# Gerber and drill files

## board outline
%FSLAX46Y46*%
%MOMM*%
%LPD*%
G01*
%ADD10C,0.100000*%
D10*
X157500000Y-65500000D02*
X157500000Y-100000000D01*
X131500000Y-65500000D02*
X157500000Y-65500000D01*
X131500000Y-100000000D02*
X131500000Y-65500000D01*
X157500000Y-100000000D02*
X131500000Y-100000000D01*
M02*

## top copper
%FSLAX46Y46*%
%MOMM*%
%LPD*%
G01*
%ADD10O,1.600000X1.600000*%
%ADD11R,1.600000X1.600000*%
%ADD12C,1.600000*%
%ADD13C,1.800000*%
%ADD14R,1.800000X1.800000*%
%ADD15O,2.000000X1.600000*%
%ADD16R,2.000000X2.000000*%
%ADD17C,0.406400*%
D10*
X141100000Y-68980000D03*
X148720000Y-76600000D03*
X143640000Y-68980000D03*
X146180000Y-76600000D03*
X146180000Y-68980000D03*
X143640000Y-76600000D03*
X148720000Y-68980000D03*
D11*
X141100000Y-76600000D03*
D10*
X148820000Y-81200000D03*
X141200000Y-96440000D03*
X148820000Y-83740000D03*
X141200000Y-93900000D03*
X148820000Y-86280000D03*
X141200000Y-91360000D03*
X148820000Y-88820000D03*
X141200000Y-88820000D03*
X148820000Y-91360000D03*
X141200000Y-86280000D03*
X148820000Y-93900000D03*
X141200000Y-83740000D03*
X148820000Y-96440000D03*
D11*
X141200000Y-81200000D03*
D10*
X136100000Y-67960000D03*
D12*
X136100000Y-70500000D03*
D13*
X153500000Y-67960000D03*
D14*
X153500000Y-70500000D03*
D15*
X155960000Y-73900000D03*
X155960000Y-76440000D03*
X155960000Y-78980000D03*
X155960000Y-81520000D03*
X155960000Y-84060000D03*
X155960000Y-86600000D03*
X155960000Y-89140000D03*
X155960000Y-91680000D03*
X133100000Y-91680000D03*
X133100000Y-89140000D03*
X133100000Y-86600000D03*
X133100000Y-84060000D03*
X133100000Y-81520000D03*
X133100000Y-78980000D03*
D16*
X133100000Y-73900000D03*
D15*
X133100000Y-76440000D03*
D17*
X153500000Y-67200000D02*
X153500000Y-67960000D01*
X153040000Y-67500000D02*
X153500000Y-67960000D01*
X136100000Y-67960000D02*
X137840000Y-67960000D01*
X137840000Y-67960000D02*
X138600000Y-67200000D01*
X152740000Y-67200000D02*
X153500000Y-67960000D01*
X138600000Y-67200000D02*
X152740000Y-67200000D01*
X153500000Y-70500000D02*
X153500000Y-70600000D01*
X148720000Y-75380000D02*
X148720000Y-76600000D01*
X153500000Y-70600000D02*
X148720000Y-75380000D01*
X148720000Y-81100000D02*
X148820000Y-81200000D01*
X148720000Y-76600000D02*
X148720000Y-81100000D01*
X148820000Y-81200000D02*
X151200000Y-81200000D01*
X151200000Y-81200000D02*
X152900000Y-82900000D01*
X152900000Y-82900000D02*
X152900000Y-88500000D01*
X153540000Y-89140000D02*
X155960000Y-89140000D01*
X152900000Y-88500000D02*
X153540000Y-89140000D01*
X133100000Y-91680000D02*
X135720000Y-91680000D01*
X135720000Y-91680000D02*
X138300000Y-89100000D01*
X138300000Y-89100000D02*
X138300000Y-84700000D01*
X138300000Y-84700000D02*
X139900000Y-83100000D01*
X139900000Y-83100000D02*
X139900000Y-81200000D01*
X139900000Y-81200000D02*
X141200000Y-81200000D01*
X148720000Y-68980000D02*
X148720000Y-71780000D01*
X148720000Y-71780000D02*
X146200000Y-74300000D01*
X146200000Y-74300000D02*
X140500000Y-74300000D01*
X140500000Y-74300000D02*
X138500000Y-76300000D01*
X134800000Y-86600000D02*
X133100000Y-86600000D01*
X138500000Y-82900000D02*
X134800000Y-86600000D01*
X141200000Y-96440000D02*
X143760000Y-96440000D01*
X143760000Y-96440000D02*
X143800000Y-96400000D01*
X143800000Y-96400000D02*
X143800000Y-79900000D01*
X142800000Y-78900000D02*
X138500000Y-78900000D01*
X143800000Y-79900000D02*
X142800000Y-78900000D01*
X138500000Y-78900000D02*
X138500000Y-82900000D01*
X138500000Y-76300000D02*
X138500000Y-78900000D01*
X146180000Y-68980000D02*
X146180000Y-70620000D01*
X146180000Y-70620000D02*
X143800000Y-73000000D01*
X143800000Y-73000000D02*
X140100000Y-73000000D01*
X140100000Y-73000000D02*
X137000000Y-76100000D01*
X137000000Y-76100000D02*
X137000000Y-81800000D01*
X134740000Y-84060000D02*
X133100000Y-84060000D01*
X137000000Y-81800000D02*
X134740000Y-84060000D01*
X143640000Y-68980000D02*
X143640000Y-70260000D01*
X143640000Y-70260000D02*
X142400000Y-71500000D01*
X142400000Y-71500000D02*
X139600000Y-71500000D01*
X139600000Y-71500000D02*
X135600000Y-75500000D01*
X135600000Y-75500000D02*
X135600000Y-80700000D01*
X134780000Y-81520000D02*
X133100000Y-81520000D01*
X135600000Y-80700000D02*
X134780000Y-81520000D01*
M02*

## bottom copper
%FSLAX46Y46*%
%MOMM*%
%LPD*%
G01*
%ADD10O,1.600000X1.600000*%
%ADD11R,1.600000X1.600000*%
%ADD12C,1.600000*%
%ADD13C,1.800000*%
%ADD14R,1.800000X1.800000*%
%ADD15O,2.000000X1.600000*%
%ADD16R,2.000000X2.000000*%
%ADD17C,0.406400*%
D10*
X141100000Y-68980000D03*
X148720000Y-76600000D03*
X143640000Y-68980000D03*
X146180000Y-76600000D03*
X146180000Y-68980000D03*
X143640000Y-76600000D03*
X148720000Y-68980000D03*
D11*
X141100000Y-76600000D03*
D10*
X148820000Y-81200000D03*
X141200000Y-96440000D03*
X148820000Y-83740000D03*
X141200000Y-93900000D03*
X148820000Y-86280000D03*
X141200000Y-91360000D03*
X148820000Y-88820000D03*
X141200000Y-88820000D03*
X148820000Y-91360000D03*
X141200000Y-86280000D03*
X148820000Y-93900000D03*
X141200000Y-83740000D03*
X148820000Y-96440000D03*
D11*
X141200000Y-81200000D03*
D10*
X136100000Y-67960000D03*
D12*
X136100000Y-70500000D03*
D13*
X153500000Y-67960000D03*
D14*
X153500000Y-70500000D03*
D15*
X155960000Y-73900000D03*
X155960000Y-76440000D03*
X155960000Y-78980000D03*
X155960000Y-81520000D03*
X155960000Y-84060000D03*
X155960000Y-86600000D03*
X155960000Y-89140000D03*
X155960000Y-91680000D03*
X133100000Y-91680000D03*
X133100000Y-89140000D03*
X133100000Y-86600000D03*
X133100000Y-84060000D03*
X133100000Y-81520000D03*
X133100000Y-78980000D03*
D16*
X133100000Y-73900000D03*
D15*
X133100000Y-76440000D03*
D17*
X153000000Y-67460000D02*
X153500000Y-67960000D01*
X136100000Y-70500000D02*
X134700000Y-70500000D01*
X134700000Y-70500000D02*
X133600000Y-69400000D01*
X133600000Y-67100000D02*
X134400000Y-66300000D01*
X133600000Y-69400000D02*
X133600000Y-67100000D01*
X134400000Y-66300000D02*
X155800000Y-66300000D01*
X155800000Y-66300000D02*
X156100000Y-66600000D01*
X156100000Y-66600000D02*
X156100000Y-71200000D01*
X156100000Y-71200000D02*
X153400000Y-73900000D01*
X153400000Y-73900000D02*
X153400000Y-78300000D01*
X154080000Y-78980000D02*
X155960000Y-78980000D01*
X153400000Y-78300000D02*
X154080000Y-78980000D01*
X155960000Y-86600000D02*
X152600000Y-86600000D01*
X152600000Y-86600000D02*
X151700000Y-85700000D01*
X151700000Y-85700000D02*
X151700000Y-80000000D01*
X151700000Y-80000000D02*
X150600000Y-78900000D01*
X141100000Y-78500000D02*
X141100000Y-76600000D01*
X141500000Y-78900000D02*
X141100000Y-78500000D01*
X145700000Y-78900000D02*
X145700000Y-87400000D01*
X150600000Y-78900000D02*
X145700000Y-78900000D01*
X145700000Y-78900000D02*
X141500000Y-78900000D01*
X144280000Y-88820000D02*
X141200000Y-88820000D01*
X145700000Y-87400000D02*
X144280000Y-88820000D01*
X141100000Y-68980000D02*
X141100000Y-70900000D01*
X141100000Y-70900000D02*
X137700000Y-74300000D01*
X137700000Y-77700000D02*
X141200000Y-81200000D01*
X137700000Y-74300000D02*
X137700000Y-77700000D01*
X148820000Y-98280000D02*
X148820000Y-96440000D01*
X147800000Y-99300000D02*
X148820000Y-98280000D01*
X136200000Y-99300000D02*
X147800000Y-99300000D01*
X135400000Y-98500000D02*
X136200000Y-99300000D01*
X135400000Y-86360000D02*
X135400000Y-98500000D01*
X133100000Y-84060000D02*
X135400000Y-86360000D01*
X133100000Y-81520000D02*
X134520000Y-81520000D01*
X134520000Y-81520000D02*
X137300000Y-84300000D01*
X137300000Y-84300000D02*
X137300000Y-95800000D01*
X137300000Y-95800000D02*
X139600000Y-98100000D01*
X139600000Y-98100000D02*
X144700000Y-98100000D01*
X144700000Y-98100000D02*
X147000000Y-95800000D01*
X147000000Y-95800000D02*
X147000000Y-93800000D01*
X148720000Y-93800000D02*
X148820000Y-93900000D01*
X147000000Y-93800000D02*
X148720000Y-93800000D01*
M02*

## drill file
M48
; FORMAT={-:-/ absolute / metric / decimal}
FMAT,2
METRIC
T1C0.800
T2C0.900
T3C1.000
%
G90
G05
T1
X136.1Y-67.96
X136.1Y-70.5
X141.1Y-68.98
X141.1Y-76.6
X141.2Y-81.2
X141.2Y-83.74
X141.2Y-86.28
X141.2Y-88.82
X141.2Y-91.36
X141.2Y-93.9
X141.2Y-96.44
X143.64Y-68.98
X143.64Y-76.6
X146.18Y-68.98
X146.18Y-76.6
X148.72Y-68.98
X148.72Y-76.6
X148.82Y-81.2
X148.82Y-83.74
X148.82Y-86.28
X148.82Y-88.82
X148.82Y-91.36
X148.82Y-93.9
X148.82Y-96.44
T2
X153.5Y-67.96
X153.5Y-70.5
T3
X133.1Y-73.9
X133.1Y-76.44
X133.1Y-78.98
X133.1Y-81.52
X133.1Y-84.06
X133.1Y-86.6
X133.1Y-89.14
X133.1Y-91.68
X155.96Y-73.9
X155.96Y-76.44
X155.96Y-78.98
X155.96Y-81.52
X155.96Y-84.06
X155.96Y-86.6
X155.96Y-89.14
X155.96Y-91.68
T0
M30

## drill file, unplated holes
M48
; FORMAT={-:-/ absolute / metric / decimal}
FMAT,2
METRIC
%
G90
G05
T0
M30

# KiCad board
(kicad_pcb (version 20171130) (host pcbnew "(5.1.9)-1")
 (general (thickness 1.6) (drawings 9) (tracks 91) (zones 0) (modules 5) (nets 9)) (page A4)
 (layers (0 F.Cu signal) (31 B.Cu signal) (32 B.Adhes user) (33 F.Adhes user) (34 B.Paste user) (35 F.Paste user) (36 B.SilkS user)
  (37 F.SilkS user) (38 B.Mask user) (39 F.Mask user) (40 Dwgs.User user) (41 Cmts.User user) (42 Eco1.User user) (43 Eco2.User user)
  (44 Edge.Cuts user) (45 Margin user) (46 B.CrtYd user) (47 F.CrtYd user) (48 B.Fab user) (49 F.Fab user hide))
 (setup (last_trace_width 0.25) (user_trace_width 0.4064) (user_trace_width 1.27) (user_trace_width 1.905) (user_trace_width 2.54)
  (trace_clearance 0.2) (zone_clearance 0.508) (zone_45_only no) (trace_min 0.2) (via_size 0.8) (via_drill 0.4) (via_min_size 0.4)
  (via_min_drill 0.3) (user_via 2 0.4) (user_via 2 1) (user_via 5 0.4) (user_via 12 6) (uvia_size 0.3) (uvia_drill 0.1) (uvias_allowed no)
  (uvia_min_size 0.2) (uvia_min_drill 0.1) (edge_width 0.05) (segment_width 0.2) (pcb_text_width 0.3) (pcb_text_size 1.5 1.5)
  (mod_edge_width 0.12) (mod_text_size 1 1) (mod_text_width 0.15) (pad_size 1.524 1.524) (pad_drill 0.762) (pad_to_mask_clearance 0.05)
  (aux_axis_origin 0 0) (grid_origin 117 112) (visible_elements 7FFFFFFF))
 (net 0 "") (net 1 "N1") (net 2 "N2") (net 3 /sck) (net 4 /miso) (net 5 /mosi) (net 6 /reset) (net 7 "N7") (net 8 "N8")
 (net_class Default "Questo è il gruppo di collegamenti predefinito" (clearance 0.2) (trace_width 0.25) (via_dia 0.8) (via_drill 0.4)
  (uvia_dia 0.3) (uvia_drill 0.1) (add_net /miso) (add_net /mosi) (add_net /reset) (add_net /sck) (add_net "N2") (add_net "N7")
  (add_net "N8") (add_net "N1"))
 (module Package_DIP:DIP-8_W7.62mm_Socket (layer F.Cu) (at 141.1 76.6 90)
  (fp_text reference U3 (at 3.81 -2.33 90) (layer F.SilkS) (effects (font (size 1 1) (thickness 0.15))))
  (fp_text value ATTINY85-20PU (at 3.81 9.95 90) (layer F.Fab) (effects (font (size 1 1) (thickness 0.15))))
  (pad 8 thru_hole oval (at 7.62 0 90) (size 1.6 1.6) (drill 0.8) (layers *.Cu *.Mask) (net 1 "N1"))
  (pad 4 thru_hole oval (at 0 7.62 90) (size 1.6 1.6) (drill 0.8) (layers *.Cu *.Mask) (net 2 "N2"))
  (pad 7 thru_hole oval (at 7.62 2.54 90) (size 1.6 1.6) (drill 0.8) (layers *.Cu *.Mask) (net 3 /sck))
  (pad 3 thru_hole oval (at 0 5.08 90) (size 1.6 1.6) (drill 0.8) (layers *.Cu *.Mask))
  (pad 6 thru_hole oval (at 7.62 5.08 90) (size 1.6 1.6) (drill 0.8) (layers *.Cu *.Mask) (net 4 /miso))
  (pad 2 thru_hole oval (at 0 2.54 90) (size 1.6 1.6) (drill 0.8) (layers *.Cu *.Mask))
  (pad 5 thru_hole oval (at 7.62 7.62 90) (size 1.6 1.6) (drill 0.8) (layers *.Cu *.Mask) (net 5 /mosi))
  (pad 1 thru_hole rect (at 0 0 90) (size 1.6 1.6) (drill 0.8) (layers *.Cu *.Mask) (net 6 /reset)))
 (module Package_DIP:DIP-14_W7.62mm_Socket (layer F.Cu) (at 141.2 81.2)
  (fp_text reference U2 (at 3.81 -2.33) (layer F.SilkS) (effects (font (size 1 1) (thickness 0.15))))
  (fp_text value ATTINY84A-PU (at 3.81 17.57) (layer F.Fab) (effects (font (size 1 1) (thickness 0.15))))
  (pad 14 thru_hole oval (at 7.62 0) (size 1.6 1.6) (drill 0.8) (layers *.Cu *.Mask) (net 2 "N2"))
  (pad 7 thru_hole oval (at 0 15.24) (size 1.6 1.6) (drill 0.8) (layers *.Cu *.Mask) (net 5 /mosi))
  (pad 13 thru_hole oval (at 7.62 2.54) (size 1.6 1.6) (drill 0.8) (layers *.Cu *.Mask))
  (pad 6 thru_hole oval (at 0 12.7) (size 1.6 1.6) (drill 0.8) (layers *.Cu *.Mask))
  (pad 12 thru_hole oval (at 7.62 5.08) (size 1.6 1.6) (drill 0.8) (layers *.Cu *.Mask))
  (pad 5 thru_hole oval (at 0 10.16) (size 1.6 1.6) (drill 0.8) (layers *.Cu *.Mask))
  (pad 11 thru_hole oval (at 7.62 7.62) (size 1.6 1.6) (drill 0.8) (layers *.Cu *.Mask))
  (pad 4 thru_hole oval (at 0 7.62) (size 1.6 1.6) (drill 0.8) (layers *.Cu *.Mask) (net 6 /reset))
  (pad 10 thru_hole oval (at 7.62 10.16) (size 1.6 1.6) (drill 0.8) (layers *.Cu *.Mask))
  (pad 3 thru_hole oval (at 0 5.08) (size 1.6 1.6) (drill 0.8) (layers *.Cu *.Mask))
  (pad 9 thru_hole oval (at 7.62 12.7) (size 1.6 1.6) (drill 0.8) (layers *.Cu *.Mask) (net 3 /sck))
  (pad 2 thru_hole oval (at 0 2.54) (size 1.6 1.6) (drill 0.8) (layers *.Cu *.Mask))
  (pad 8 thru_hole oval (at 7.62 15.24) (size 1.6 1.6) (drill 0.8) (layers *.Cu *.Mask) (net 4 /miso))
  (pad 1 thru_hole rect (at 0 0) (size 1.6 1.6) (drill 0.8) (layers *.Cu *.Mask) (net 1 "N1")))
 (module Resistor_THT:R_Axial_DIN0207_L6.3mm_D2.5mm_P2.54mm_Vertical (layer F.Cu) (at 136.1 70.5 90)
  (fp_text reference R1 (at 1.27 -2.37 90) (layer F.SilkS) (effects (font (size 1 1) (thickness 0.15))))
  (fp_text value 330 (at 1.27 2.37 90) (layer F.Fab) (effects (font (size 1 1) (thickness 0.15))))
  (pad 2 thru_hole oval (at 2.54 0 90) (size 1.6 1.6) (drill 0.8) (layers *.Cu *.Mask) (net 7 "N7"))
  (pad 1 thru_hole circle (at 0 0 90) (size 1.6 1.6) (drill 0.8) (layers *.Cu *.Mask) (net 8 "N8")))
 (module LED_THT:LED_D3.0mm (layer F.Cu) (at 153.5 70.5 90)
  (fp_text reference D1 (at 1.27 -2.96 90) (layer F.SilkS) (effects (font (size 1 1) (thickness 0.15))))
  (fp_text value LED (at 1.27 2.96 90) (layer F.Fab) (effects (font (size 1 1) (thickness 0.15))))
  (pad 2 thru_hole circle (at 2.54 0 90) (size 1.8 1.8) (drill 0.9) (layers *.Cu *.Mask) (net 7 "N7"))
  (pad 1 thru_hole rect (at 0 0 90) (size 1.8 1.8) (drill 0.9) (layers *.Cu *.Mask) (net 2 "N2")))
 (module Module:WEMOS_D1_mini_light (layer F.Cu) (at 133.1 73.9)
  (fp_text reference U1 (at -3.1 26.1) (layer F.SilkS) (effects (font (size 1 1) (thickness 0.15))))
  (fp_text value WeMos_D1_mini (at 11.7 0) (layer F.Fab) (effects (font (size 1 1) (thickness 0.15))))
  (pad 16 thru_hole oval (at 22.86 0) (size 2 1.6) (drill 1) (layers *.Cu *.Mask))
  (pad 15 thru_hole oval (at 22.86 2.54) (size 2 1.6) (drill 1) (layers *.Cu *.Mask))
  (pad 14 thru_hole oval (at 22.86 5.08) (size 2 1.6) (drill 1) (layers *.Cu *.Mask) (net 8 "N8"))
  (pad 13 thru_hole oval (at 22.86 7.62) (size 2 1.6) (drill 1) (layers *.Cu *.Mask))
  (pad 12 thru_hole oval (at 22.86 10.16) (size 2 1.6) (drill 1) (layers *.Cu *.Mask))
  (pad 11 thru_hole oval (at 22.86 12.7) (size 2 1.6) (drill 1) (layers *.Cu *.Mask) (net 6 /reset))
  (pad 10 thru_hole oval (at 22.86 15.24) (size 2 1.6) (drill 1) (layers *.Cu *.Mask) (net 2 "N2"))
  (pad 9 thru_hole oval (at 22.86 17.78) (size 2 1.6) (drill 1) (layers *.Cu *.Mask))
  (pad 8 thru_hole oval (at 0 17.78) (size 2 1.6) (drill 1) (layers *.Cu *.Mask) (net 1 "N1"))
  (pad 7 thru_hole oval (at 0 15.24) (size 2 1.6) (drill 1) (layers *.Cu *.Mask))
  (pad 6 thru_hole oval (at 0 12.7) (size 2 1.6) (drill 1) (layers *.Cu *.Mask) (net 5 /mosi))
  (pad 5 thru_hole oval (at 0 10.16) (size 2 1.6) (drill 1) (layers *.Cu *.Mask) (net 4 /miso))
  (pad 4 thru_hole oval (at 0 7.62) (size 2 1.6) (drill 1) (layers *.Cu *.Mask) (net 3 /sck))
  (pad 3 thru_hole oval (at 0 5.08) (size 2 1.6) (drill 1) (layers *.Cu *.Mask))
  (pad 1 thru_hole rect (at 0 0) (size 2 2) (drill 1) (layers *.Cu *.Mask))
  (pad 2 thru_hole oval (at 0 2.54) (size 2 1.6) (drill 1) (layers *.Cu *.Mask)))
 (gr_line (start 157.5 65.5) (end 157.5 100) (layer Edge.Cuts) (width 0.1))
 (gr_line (start 131.5 65.5) (end 157.5 65.5) (layer Edge.Cuts) (width 0.1))
 (gr_line (start 131.5 100) (end 131.5 65.5) (layer Edge.Cuts) (width 0.1))
 (gr_line (start 157.5 100) (end 131.5 100) (layer Edge.Cuts) (width 0.1))
 (segment (start 153 67.46) (end 153.5 67.96) (width 0.4064) (layer B.Cu) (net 7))
 (segment (start 153.5 67.2) (end 153.5 67.96) (width 0.4064) (layer F.Cu) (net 7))
 (segment (start 153.04 67.5) (end 153.5 67.96) (width 0.4064) (layer F.Cu) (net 7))
 (segment (start 136.1 67.96) (end 137.84 67.96) (width 0.4064) (layer F.Cu) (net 7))
 (segment (start 137.84 67.96) (end 138.6 67.2) (width 0.4064) (layer F.Cu) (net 7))
 (segment (start 152.74 67.2) (end 153.5 67.96) (width 0.4064) (layer F.Cu) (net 7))
 (segment (start 138.6 67.2) (end 152.74 67.2) (width 0.4064) (layer F.Cu) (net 7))
 (segment (start 153.5 70.5) (end 153.5 70.6) (width 0.4064) (layer F.Cu) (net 2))
 (segment (start 148.72 75.38) (end 148.72 76.6) (width 0.4064) (layer F.Cu) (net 2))
 (segment (start 153.5 70.6) (end 148.72 75.38) (width 0.4064) (layer F.Cu) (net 2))
 (segment (start 148.72 81.1) (end 148.82 81.2) (width 0.4064) (layer F.Cu) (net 2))
 (segment (start 148.72 76.6) (end 148.72 81.1) (width 0.4064) (layer F.Cu) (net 2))
 (segment (start 148.82 81.2) (end 151.2 81.2) (width 0.4064) (layer F.Cu) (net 2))
 (segment (start 151.2 81.2) (end 152.9 82.9) (width 0.4064) (layer F.Cu) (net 2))
 (segment (start 152.9 82.9) (end 152.9 88.5) (width 0.4064) (layer F.Cu) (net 2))
 (segment (start 153.54 89.14) (end 155.96 89.14) (width 0.4064) (layer F.Cu) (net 2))
 (segment (start 152.9 88.5) (end 153.54 89.14) (width 0.4064) (layer F.Cu) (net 2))
 (segment (start 136.1 70.5) (end 134.7 70.5) (width 0.4064) (layer B.Cu) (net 8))
 (segment (start 134.7 70.5) (end 133.6 69.4) (width 0.4064) (layer B.Cu) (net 8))
 (segment (start 133.6 67.1) (end 134.4 66.3) (width 0.4064) (layer B.Cu) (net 8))
 (segment (start 133.6 69.4) (end 133.6 67.1) (width 0.4064) (layer B.Cu) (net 8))
 (segment (start 134.4 66.3) (end 155.8 66.3) (width 0.4064) (layer B.Cu) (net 8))
 (segment (start 155.8 66.3) (end 156.1 66.6) (width 0.4064) (layer B.Cu) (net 8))
 (segment (start 156.1 66.6) (end 156.1 71.2) (width 0.4064) (layer B.Cu) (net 8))
 (segment (start 156.1 71.2) (end 153.4 73.9) (width 0.4064) (layer B.Cu) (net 8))
 (segment (start 153.4 73.9) (end 153.4 78.3) (width 0.4064) (layer B.Cu) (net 8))
 (segment (start 154.08 78.98) (end 155.96 78.98) (width 0.4064) (layer B.Cu) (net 8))
 (segment (start 153.4 78.3) (end 154.08 78.98) (width 0.4064) (layer B.Cu) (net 8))
 (segment (start 155.96 86.6) (end 152.6 86.6) (width 0.4064) (layer B.Cu) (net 6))
 (segment (start 152.6 86.6) (end 151.7 85.7) (width 0.4064) (layer B.Cu) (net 6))
 (segment (start 151.7 85.7) (end 151.7 80) (width 0.4064) (layer B.Cu) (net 6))
 (segment (start 151.7 80) (end 150.6 78.9) (width 0.4064) (layer B.Cu) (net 6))
 (segment (start 141.1 78.5) (end 141.1 76.6) (width 0.4064) (layer B.Cu) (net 6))
 (segment (start 141.5 78.9) (end 141.1 78.5) (width 0.4064) (layer B.Cu) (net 6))
 (segment (start 145.7 78.9) (end 145.7 87.4) (width 0.4064) (layer B.Cu) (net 6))
 (segment (start 150.6 78.9) (end 145.7 78.9) (width 0.4064) (layer B.Cu) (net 6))
 (segment (start 145.7 78.9) (end 141.5 78.9) (width 0.4064) (layer B.Cu) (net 6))
 (segment (start 144.28 88.82) (end 141.2 88.82) (width 0.4064) (layer B.Cu) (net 6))
 (segment (start 145.7 87.4) (end 144.28 88.82) (width 0.4064) (layer B.Cu) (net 6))
 (segment (start 133.1 91.68) (end 135.72 91.68) (width 0.4064) (layer F.Cu) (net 1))
 (segment (start 135.72 91.68) (end 138.3 89.1) (width 0.4064) (layer F.Cu) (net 1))
 (segment (start 138.3 89.1) (end 138.3 84.7) (width 0.4064) (layer F.Cu) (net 1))
 (segment (start 138.3 84.7) (end 139.9 83.1) (width 0.4064) (layer F.Cu) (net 1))
 (segment (start 139.9 83.1) (end 139.9 81.2) (width 0.4064) (layer F.Cu) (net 1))
 (segment (start 139.9 81.2) (end 141.2 81.2) (width 0.4064) (layer F.Cu) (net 1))
 (segment (start 141.1 68.98) (end 141.1 70.9) (width 0.4064) (layer B.Cu) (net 1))
 (segment (start 141.1 70.9) (end 137.7 74.3) (width 0.4064) (layer B.Cu) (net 1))
 (segment (start 137.7 77.7) (end 141.2 81.2) (width 0.4064) (layer B.Cu) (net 1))
 (segment (start 137.7 74.3) (end 137.7 77.7) (width 0.4064) (layer B.Cu) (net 1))
 (segment (start 148.72 68.98) (end 148.72 71.78) (width 0.4064) (layer F.Cu) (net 5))
 (segment (start 148.72 71.78) (end 146.2 74.3) (width 0.4064) (layer F.Cu) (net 5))
 (segment (start 146.2 74.3) (end 140.5 74.3) (width 0.4064) (layer F.Cu) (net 5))
 (segment (start 140.5 74.3) (end 138.5 76.3) (width 0.4064) (layer F.Cu) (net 5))
 (segment (start 134.8 86.6) (end 133.1 86.6) (width 0.4064) (layer F.Cu) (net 5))
 (segment (start 138.5 82.9) (end 134.8 86.6) (width 0.4064) (layer F.Cu) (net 5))
 (segment (start 141.2 96.44) (end 143.76 96.44) (width 0.4064) (layer F.Cu) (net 5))
 (segment (start 143.76 96.44) (end 143.8 96.4) (width 0.4064) (layer F.Cu) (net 5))
 (segment (start 143.8 96.4) (end 143.8 79.9) (width 0.4064) (layer F.Cu) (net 5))
 (segment (start 142.8 78.9) (end 138.5 78.9) (width 0.4064) (layer F.Cu) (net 5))
 (segment (start 143.8 79.9) (end 142.8 78.9) (width 0.4064) (layer F.Cu) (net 5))
 (segment (start 138.5 78.9) (end 138.5 82.9) (width 0.4064) (layer F.Cu) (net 5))
 (segment (start 138.5 76.3) (end 138.5 78.9) (width 0.4064) (layer F.Cu) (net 5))
 (segment (start 146.18 68.98) (end 146.18 70.62) (width 0.4064) (layer F.Cu) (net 4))
 (segment (start 146.18 70.62) (end 143.8 73) (width 0.4064) (layer F.Cu) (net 4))
 (segment (start 143.8 73) (end 140.1 73) (width 0.4064) (layer F.Cu) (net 4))
 (segment (start 140.1 73) (end 137 76.1) (width 0.4064) (layer F.Cu) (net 4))
 (segment (start 137 76.1) (end 137 81.8) (width 0.4064) (layer F.Cu) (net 4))
 (segment (start 134.74 84.06) (end 133.1 84.06) (width 0.4064) (layer F.Cu) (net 4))
 (segment (start 137 81.8) (end 134.74 84.06) (width 0.4064) (layer F.Cu) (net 4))
 (segment (start 148.82 98.28) (end 148.82 96.44) (width 0.4064) (layer B.Cu) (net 4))
 (segment (start 147.8 99.3) (end 148.82 98.28) (width 0.4064) (layer B.Cu) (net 4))
 (segment (start 136.2 99.3) (end 147.8 99.3) (width 0.4064) (layer B.Cu) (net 4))
 (segment (start 135.4 98.5) (end 136.2 99.3) (width 0.4064) (layer B.Cu) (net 4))
 (segment (start 135.4 86.36) (end 135.4 98.5) (width 0.4064) (layer B.Cu) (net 4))
 (segment (start 133.1 84.06) (end 135.4 86.36) (width 0.4064) (layer B.Cu) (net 4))
 (segment (start 143.64 68.98) (end 143.64 70.26) (width 0.4064) (layer F.Cu) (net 3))
 (segment (start 143.64 70.26) (end 142.4 71.5) (width 0.4064) (layer F.Cu) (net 3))
 (segment (start 142.4 71.5) (end 139.6 71.5) (width 0.4064) (layer F.Cu) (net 3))
 (segment (start 139.6 71.5) (end 135.6 75.5) (width 0.4064) (layer F.Cu) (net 3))
 (segment (start 135.6 75.5) (end 135.6 80.7) (width 0.4064) (layer F.Cu) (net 3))
 (segment (start 134.78 81.52) (end 133.1 81.52) (width 0.4064) (layer F.Cu) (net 3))
 (segment (start 135.6 80.7) (end 134.78 81.52) (width 0.4064) (layer F.Cu) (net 3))
 (segment (start 133.1 81.52) (end 134.52 81.52) (width 0.4064) (layer B.Cu) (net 3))
 (segment (start 134.52 81.52) (end 137.3 84.3) (width 0.4064) (layer B.Cu) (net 3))
 (segment (start 137.3 84.3) (end 137.3 95.8) (width 0.4064) (layer B.Cu) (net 3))
 (segment (start 137.3 95.8) (end 139.6 98.1) (width 0.4064) (layer B.Cu) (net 3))
 (segment (start 139.6 98.1) (end 144.7 98.1) (width 0.4064) (layer B.Cu) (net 3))
 (segment (start 144.7 98.1) (end 147 95.8) (width 0.4064) (layer B.Cu) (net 3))
 (segment (start 147 95.8) (end 147 93.8) (width 0.4064) (layer B.Cu) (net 3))
 (segment (start 148.72 93.8) (end 148.82 93.9) (width 0.4064) (layer B.Cu) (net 3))
 (segment (start 147 93.8) (end 148.72 93.8) (width 0.4064) (layer B.Cu) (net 3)))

